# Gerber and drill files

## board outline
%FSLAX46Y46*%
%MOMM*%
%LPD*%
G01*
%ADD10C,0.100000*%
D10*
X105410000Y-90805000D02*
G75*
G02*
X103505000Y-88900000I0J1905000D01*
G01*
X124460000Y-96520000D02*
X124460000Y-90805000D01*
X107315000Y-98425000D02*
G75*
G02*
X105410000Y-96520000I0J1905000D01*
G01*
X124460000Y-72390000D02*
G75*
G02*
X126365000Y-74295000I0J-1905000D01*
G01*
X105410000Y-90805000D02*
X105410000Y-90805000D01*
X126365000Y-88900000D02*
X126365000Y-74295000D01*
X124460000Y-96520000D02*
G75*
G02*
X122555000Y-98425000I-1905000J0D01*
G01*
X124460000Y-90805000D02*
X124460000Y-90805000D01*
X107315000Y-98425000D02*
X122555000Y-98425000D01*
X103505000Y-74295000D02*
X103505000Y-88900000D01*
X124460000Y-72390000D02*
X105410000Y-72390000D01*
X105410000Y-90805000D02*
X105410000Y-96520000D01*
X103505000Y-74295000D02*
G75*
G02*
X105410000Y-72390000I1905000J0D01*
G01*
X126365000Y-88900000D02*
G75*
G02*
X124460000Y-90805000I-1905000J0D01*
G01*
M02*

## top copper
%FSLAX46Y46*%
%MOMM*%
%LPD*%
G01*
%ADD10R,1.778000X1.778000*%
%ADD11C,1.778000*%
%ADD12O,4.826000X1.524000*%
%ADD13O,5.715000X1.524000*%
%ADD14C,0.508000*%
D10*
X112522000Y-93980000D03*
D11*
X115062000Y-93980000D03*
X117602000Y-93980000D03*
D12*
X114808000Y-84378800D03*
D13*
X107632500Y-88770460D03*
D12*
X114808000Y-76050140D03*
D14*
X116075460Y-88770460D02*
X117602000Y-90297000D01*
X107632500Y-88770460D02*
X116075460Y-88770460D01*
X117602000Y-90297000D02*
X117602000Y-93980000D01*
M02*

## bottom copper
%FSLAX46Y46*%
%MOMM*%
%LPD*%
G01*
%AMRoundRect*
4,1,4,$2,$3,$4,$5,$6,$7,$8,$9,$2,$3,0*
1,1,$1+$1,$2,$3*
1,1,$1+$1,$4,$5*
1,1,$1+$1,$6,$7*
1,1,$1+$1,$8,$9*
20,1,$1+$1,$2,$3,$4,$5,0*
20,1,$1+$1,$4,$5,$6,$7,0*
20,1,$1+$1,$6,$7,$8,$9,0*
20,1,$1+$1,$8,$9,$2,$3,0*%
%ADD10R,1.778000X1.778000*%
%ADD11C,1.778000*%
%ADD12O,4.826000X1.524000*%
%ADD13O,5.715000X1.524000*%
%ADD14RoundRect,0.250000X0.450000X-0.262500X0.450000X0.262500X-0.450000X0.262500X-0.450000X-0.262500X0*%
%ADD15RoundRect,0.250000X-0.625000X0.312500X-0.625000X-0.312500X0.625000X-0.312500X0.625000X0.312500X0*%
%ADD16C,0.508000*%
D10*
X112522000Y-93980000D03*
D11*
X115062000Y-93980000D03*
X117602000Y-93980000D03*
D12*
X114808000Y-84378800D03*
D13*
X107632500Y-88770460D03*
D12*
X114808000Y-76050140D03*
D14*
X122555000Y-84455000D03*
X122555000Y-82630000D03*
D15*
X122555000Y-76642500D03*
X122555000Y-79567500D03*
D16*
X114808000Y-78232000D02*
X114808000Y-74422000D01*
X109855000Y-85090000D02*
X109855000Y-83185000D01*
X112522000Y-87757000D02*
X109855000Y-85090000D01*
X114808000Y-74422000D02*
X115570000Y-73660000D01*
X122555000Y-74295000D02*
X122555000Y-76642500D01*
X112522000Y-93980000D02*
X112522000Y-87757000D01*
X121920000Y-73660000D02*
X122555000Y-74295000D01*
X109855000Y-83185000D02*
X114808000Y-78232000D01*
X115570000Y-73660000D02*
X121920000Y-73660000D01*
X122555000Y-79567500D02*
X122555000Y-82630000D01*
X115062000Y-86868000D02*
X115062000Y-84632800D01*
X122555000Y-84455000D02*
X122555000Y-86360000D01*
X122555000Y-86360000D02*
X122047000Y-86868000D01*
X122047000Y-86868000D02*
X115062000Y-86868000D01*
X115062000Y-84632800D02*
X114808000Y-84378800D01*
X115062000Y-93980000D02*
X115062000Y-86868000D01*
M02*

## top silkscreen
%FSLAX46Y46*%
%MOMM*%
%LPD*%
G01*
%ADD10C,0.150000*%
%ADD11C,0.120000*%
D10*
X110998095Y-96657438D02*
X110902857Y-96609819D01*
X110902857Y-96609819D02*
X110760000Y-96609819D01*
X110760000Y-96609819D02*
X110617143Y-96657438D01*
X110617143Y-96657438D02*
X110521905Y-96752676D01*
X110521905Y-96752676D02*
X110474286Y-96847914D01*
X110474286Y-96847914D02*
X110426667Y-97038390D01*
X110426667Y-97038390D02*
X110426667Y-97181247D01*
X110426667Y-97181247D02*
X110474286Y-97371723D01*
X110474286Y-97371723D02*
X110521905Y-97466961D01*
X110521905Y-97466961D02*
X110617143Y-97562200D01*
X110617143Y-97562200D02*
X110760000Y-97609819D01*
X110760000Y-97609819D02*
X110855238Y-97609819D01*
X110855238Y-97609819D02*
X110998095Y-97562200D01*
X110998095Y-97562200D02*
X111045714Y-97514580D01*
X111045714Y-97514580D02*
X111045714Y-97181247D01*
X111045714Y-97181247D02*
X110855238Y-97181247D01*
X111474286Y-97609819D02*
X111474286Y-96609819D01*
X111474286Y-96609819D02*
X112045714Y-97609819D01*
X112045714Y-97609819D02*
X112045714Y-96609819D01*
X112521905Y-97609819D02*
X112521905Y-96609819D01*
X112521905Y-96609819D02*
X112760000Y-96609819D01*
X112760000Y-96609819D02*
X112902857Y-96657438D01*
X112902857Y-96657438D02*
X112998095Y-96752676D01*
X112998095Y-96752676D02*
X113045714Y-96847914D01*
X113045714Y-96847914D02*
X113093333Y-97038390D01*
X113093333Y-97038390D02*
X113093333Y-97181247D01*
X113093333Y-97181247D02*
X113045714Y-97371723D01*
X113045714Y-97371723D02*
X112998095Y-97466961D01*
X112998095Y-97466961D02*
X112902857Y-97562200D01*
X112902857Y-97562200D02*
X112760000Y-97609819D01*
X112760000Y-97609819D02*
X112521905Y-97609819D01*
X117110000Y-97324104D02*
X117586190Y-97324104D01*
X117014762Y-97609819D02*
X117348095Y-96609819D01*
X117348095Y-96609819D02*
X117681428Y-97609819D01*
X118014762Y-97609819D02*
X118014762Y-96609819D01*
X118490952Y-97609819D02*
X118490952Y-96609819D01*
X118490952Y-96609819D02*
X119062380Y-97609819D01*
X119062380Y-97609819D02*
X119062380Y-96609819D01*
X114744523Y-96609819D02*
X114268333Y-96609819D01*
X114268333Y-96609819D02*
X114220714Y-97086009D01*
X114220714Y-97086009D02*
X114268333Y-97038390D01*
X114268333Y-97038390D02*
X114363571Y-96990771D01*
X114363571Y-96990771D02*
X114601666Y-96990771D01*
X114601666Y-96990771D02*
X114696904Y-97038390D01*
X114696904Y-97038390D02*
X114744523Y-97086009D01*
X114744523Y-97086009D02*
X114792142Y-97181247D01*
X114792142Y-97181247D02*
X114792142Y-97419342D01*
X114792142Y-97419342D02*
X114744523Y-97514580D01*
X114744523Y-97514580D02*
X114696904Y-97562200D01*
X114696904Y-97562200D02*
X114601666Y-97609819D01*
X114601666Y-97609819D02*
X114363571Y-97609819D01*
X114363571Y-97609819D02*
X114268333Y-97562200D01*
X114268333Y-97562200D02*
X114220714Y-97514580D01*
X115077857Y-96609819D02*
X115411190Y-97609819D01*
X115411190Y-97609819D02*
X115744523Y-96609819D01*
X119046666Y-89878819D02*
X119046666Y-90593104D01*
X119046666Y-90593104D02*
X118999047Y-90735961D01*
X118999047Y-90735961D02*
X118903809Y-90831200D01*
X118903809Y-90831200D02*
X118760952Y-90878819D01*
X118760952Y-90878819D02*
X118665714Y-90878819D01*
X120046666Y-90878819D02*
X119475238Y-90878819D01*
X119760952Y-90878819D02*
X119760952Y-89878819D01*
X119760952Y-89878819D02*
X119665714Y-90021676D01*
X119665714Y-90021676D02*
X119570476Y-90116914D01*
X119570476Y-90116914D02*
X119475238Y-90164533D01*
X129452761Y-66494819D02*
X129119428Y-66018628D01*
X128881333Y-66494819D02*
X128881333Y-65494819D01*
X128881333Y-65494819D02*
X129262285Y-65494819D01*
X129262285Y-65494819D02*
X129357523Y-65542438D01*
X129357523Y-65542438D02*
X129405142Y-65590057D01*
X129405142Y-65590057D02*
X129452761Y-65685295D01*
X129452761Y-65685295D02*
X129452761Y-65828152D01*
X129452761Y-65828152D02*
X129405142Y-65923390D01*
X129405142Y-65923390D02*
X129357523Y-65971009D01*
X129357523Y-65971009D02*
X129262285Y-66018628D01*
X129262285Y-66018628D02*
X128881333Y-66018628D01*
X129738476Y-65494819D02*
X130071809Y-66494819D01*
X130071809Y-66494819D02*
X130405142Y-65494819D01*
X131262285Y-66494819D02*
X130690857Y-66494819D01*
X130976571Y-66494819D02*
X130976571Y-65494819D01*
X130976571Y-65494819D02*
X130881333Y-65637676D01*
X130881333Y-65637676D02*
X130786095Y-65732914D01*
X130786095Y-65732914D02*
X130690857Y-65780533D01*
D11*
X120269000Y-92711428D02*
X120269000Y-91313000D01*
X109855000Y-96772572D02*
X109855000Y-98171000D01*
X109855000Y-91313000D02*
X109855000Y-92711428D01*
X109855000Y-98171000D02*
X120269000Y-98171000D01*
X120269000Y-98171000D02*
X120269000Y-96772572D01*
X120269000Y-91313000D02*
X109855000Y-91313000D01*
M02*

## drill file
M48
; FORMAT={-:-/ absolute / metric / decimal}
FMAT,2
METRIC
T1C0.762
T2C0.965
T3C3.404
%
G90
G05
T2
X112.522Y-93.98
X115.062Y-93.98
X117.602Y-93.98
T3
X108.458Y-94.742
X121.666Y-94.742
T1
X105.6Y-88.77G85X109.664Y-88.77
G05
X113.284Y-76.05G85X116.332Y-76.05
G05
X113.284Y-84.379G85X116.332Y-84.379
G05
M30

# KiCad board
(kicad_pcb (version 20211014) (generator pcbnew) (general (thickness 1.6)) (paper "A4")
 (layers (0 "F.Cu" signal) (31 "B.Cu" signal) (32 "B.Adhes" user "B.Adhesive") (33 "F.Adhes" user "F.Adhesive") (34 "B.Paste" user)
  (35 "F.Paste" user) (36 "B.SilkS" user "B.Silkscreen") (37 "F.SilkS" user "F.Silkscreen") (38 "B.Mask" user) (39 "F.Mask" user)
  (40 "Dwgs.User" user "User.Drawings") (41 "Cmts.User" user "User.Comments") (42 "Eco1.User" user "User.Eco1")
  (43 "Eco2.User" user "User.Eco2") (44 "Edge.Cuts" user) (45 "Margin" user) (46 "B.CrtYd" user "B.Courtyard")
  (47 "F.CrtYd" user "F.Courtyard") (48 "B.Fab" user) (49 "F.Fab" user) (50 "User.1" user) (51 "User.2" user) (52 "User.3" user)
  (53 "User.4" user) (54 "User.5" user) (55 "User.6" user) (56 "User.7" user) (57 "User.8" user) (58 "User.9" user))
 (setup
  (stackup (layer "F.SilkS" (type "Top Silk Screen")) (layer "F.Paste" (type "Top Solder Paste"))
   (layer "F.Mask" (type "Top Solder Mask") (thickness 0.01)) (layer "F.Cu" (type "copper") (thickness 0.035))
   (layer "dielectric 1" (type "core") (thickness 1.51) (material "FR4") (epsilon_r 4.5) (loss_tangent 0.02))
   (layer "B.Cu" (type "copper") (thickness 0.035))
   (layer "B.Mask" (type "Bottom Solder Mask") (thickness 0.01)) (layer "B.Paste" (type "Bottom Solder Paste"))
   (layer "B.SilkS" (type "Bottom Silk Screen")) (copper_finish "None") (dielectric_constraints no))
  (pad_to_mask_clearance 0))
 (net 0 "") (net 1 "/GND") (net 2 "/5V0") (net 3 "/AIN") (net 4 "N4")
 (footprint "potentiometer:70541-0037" (layer "F.Cu") (at 112.522 93.98 180)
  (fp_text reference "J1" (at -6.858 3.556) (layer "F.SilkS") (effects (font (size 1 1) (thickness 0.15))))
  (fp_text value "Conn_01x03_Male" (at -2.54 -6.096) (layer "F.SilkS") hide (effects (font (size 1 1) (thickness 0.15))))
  (fp_line (start -7.747 1.268572) (end -7.747 2.667) (layer "F.SilkS") (width 0.12))
  (fp_line (start 2.667 -2.792572) (end 2.667 -4.191) (layer "F.SilkS") (width 0.12))
  (fp_line (start 2.667 2.667) (end 2.667 1.268572) (layer "F.SilkS") (width 0.12))
  (fp_line (start 2.667 -4.191) (end -7.747 -4.191) (layer "F.SilkS") (width 0.12))
  (fp_line (start -7.747 -4.191) (end -7.747 -2.792572) (layer "F.SilkS") (width 0.12))
  (fp_line (start -7.747 2.667) (end 2.667 2.667) (layer "F.SilkS") (width 0.12))
  (pad "" np_thru_hole circle (at -9.144 -0.762 180) (size 3.4036 3.4036) (drill 3.4036) (layers *.Cu *.Mask))
  (pad "" np_thru_hole circle (at 4.064 -0.762 180) (size 3.4036 3.4036) (drill 3.4036) (layers *.Cu *.Mask))
  (pad "1" thru_hole rect (at 0 0 180) (size 1.778 1.778) (drill 0.9652) (layers *.Cu *.Mask) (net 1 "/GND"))
  (pad "2" thru_hole circle (at -2.54 0 180) (size 1.778 1.778) (drill 0.9652) (layers *.Cu *.Mask) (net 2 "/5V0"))
  (pad "3" thru_hole circle (at -5.08 0 180) (size 1.778 1.778) (drill 0.9652) (layers *.Cu *.Mask) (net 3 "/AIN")))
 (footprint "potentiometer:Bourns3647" (layer "F.Cu") (at 114.808 78.74)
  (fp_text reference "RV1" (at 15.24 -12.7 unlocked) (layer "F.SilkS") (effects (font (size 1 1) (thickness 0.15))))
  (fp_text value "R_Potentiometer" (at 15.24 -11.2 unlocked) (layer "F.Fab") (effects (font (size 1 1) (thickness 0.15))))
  (pad "1" thru_hole oval (at 0 5.6388) (size 4.826 1.524) (drill oval 3.81 0.762) (layers *.Cu *.Mask) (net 2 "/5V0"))
  (pad "2" thru_hole oval (at -7.1755 10.03046) (size 5.715 1.524) (drill oval 4.826 0.762) (layers *.Cu *.Mask) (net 3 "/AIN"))
  (pad "3" thru_hole oval (at 0 -2.68986) (size 4.826 1.524) (drill oval 3.81 0.762) (layers *.Cu *.Mask) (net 1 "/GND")))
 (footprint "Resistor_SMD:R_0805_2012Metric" (layer "B.Cu") (at 122.555 83.5425 90)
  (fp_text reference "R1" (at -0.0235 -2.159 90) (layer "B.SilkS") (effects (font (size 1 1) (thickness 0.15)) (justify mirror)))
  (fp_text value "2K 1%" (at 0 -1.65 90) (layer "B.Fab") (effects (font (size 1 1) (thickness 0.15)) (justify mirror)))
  (pad "1" smd roundrect (at -0.9125 0 90) (size 1.025 1.4) (layers "B.Cu" "B.Paste" "B.Mask") (roundrect_rratio 0.243902) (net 2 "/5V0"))
  (pad "2" smd roundrect (at 0.9125 0 90) (size 1.025 1.4) (layers "B.Cu" "B.Paste" "B.Mask") (roundrect_rratio 0.243902) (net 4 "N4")))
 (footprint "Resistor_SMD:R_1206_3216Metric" (layer "B.Cu") (at 122.555 78.105 -90)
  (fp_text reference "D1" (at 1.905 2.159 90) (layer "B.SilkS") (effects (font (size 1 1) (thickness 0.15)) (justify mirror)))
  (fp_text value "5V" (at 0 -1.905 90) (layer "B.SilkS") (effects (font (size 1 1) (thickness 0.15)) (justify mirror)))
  (pad "1" smd roundrect (at -1.4625 0 270) (size 1.125 1.75) (layers "B.Cu" "B.Paste" "B.Mask") (roundrect_rratio 0.222222) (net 1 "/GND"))
  (pad "2" smd roundrect (at 1.4625 0 270) (size 1.125 1.75) (layers "B.Cu" "B.Paste" "B.Mask") (roundrect_rratio 0.222222) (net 4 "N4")))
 (gr_arc (start 105.41 90.805) (mid 104.062962 90.247038) (end 103.505 88.9) (layer "Edge.Cuts") (width 0.1))
 (gr_line (start 124.46 96.52) (end 124.46 90.805) (layer "Edge.Cuts") (width 0.1))
 (gr_arc (start 107.315 98.425) (mid 105.967962 97.867038) (end 105.41 96.52) (layer "Edge.Cuts") (width 0.1))
 (gr_arc (start 124.46 72.39) (mid 125.807038 72.947962) (end 126.365 74.295) (layer "Edge.Cuts") (width 0.1))
 (gr_line (start 105.41 90.805) (end 105.41 90.805) (layer "Edge.Cuts") (width 0.1))
 (gr_line (start 126.365 88.9) (end 126.365 74.295) (layer "Edge.Cuts") (width 0.1))
 (gr_arc (start 124.46 96.52) (mid 123.902038 97.867038) (end 122.555 98.425) (layer "Edge.Cuts") (width 0.1))
 (gr_line (start 124.46 90.805) (end 124.46 90.805) (layer "Edge.Cuts") (width 0.1))
 (gr_line (start 107.315 98.425) (end 122.555 98.425) (layer "Edge.Cuts") (width 0.1))
 (gr_line (start 103.505 74.295) (end 103.505 88.9) (layer "Edge.Cuts") (width 0.1))
 (gr_line (start 124.46 72.39) (end 105.41 72.39) (layer "Edge.Cuts") (width 0.1))
 (gr_line (start 105.41 90.805) (end 105.41 96.52) (layer "Edge.Cuts") (width 0.1))
 (gr_arc (start 103.505 74.295) (mid 104.062962 72.947962) (end 105.41 72.39) (layer "Edge.Cuts") (width 0.1))
 (gr_arc (start 126.365 88.9) (mid 125.807038 90.247038) (end 124.46 90.805) (layer "Edge.Cuts") (width 0.1))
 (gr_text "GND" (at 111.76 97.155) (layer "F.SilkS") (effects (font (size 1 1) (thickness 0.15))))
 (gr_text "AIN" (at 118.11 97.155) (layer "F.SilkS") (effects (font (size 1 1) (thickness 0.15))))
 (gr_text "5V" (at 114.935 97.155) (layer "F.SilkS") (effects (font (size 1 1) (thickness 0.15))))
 (segment (start 114.808 78.232) (end 114.808 74.422) (width 0.508) (layer "B.Cu") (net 1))
 (segment (start 109.855 85.09) (end 109.855 83.185) (width 0.508) (layer "B.Cu") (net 1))
 (segment (start 112.522 87.757) (end 109.855 85.09) (width 0.508) (layer "B.Cu") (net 1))
 (segment (start 114.808 74.422) (end 115.57 73.66) (width 0.508) (layer "B.Cu") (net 1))
 (segment (start 122.555 74.295) (end 122.555 76.6425) (width 0.508) (layer "B.Cu") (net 1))
 (segment (start 112.522 93.98) (end 112.522 87.757) (width 0.508) (layer "B.Cu") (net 1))
 (segment (start 121.92 73.66) (end 122.555 74.295) (width 0.508) (layer "B.Cu") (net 1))
 (segment (start 109.855 83.185) (end 114.808 78.232) (width 0.508) (layer "B.Cu") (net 1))
 (segment (start 115.57 73.66) (end 121.92 73.66) (width 0.508) (layer "B.Cu") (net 1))
 (segment (start 122.555 79.5675) (end 122.555 82.63) (width 0.508) (layer "B.Cu") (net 4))
 (segment (start 115.062 86.868) (end 115.062 84.6328) (width 0.508) (layer "B.Cu") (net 2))
 (segment (start 122.555 84.455) (end 122.555 86.36) (width 0.508) (layer "B.Cu") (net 2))
 (segment (start 122.555 86.36) (end 122.047 86.868) (width 0.508) (layer "B.Cu") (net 2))
 (segment (start 122.047 86.868) (end 115.062 86.868) (width 0.508) (layer "B.Cu") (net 2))
 (segment (start 115.062 84.6328) (end 114.808 84.3788) (width 0.508) (layer "B.Cu") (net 2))
 (segment (start 115.062 93.98) (end 115.062 86.868) (width 0.508) (layer "B.Cu") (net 2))
 (segment (start 116.07546 88.77046) (end 117.602 90.297) (width 0.508) (layer "F.Cu") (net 3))
 (segment (start 107.6325 88.77046) (end 116.07546 88.77046) (width 0.508) (layer "F.Cu") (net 3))
 (segment (start 117.602 90.297) (end 117.602 93.98) (width 0.508) (layer "F.Cu") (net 3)))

